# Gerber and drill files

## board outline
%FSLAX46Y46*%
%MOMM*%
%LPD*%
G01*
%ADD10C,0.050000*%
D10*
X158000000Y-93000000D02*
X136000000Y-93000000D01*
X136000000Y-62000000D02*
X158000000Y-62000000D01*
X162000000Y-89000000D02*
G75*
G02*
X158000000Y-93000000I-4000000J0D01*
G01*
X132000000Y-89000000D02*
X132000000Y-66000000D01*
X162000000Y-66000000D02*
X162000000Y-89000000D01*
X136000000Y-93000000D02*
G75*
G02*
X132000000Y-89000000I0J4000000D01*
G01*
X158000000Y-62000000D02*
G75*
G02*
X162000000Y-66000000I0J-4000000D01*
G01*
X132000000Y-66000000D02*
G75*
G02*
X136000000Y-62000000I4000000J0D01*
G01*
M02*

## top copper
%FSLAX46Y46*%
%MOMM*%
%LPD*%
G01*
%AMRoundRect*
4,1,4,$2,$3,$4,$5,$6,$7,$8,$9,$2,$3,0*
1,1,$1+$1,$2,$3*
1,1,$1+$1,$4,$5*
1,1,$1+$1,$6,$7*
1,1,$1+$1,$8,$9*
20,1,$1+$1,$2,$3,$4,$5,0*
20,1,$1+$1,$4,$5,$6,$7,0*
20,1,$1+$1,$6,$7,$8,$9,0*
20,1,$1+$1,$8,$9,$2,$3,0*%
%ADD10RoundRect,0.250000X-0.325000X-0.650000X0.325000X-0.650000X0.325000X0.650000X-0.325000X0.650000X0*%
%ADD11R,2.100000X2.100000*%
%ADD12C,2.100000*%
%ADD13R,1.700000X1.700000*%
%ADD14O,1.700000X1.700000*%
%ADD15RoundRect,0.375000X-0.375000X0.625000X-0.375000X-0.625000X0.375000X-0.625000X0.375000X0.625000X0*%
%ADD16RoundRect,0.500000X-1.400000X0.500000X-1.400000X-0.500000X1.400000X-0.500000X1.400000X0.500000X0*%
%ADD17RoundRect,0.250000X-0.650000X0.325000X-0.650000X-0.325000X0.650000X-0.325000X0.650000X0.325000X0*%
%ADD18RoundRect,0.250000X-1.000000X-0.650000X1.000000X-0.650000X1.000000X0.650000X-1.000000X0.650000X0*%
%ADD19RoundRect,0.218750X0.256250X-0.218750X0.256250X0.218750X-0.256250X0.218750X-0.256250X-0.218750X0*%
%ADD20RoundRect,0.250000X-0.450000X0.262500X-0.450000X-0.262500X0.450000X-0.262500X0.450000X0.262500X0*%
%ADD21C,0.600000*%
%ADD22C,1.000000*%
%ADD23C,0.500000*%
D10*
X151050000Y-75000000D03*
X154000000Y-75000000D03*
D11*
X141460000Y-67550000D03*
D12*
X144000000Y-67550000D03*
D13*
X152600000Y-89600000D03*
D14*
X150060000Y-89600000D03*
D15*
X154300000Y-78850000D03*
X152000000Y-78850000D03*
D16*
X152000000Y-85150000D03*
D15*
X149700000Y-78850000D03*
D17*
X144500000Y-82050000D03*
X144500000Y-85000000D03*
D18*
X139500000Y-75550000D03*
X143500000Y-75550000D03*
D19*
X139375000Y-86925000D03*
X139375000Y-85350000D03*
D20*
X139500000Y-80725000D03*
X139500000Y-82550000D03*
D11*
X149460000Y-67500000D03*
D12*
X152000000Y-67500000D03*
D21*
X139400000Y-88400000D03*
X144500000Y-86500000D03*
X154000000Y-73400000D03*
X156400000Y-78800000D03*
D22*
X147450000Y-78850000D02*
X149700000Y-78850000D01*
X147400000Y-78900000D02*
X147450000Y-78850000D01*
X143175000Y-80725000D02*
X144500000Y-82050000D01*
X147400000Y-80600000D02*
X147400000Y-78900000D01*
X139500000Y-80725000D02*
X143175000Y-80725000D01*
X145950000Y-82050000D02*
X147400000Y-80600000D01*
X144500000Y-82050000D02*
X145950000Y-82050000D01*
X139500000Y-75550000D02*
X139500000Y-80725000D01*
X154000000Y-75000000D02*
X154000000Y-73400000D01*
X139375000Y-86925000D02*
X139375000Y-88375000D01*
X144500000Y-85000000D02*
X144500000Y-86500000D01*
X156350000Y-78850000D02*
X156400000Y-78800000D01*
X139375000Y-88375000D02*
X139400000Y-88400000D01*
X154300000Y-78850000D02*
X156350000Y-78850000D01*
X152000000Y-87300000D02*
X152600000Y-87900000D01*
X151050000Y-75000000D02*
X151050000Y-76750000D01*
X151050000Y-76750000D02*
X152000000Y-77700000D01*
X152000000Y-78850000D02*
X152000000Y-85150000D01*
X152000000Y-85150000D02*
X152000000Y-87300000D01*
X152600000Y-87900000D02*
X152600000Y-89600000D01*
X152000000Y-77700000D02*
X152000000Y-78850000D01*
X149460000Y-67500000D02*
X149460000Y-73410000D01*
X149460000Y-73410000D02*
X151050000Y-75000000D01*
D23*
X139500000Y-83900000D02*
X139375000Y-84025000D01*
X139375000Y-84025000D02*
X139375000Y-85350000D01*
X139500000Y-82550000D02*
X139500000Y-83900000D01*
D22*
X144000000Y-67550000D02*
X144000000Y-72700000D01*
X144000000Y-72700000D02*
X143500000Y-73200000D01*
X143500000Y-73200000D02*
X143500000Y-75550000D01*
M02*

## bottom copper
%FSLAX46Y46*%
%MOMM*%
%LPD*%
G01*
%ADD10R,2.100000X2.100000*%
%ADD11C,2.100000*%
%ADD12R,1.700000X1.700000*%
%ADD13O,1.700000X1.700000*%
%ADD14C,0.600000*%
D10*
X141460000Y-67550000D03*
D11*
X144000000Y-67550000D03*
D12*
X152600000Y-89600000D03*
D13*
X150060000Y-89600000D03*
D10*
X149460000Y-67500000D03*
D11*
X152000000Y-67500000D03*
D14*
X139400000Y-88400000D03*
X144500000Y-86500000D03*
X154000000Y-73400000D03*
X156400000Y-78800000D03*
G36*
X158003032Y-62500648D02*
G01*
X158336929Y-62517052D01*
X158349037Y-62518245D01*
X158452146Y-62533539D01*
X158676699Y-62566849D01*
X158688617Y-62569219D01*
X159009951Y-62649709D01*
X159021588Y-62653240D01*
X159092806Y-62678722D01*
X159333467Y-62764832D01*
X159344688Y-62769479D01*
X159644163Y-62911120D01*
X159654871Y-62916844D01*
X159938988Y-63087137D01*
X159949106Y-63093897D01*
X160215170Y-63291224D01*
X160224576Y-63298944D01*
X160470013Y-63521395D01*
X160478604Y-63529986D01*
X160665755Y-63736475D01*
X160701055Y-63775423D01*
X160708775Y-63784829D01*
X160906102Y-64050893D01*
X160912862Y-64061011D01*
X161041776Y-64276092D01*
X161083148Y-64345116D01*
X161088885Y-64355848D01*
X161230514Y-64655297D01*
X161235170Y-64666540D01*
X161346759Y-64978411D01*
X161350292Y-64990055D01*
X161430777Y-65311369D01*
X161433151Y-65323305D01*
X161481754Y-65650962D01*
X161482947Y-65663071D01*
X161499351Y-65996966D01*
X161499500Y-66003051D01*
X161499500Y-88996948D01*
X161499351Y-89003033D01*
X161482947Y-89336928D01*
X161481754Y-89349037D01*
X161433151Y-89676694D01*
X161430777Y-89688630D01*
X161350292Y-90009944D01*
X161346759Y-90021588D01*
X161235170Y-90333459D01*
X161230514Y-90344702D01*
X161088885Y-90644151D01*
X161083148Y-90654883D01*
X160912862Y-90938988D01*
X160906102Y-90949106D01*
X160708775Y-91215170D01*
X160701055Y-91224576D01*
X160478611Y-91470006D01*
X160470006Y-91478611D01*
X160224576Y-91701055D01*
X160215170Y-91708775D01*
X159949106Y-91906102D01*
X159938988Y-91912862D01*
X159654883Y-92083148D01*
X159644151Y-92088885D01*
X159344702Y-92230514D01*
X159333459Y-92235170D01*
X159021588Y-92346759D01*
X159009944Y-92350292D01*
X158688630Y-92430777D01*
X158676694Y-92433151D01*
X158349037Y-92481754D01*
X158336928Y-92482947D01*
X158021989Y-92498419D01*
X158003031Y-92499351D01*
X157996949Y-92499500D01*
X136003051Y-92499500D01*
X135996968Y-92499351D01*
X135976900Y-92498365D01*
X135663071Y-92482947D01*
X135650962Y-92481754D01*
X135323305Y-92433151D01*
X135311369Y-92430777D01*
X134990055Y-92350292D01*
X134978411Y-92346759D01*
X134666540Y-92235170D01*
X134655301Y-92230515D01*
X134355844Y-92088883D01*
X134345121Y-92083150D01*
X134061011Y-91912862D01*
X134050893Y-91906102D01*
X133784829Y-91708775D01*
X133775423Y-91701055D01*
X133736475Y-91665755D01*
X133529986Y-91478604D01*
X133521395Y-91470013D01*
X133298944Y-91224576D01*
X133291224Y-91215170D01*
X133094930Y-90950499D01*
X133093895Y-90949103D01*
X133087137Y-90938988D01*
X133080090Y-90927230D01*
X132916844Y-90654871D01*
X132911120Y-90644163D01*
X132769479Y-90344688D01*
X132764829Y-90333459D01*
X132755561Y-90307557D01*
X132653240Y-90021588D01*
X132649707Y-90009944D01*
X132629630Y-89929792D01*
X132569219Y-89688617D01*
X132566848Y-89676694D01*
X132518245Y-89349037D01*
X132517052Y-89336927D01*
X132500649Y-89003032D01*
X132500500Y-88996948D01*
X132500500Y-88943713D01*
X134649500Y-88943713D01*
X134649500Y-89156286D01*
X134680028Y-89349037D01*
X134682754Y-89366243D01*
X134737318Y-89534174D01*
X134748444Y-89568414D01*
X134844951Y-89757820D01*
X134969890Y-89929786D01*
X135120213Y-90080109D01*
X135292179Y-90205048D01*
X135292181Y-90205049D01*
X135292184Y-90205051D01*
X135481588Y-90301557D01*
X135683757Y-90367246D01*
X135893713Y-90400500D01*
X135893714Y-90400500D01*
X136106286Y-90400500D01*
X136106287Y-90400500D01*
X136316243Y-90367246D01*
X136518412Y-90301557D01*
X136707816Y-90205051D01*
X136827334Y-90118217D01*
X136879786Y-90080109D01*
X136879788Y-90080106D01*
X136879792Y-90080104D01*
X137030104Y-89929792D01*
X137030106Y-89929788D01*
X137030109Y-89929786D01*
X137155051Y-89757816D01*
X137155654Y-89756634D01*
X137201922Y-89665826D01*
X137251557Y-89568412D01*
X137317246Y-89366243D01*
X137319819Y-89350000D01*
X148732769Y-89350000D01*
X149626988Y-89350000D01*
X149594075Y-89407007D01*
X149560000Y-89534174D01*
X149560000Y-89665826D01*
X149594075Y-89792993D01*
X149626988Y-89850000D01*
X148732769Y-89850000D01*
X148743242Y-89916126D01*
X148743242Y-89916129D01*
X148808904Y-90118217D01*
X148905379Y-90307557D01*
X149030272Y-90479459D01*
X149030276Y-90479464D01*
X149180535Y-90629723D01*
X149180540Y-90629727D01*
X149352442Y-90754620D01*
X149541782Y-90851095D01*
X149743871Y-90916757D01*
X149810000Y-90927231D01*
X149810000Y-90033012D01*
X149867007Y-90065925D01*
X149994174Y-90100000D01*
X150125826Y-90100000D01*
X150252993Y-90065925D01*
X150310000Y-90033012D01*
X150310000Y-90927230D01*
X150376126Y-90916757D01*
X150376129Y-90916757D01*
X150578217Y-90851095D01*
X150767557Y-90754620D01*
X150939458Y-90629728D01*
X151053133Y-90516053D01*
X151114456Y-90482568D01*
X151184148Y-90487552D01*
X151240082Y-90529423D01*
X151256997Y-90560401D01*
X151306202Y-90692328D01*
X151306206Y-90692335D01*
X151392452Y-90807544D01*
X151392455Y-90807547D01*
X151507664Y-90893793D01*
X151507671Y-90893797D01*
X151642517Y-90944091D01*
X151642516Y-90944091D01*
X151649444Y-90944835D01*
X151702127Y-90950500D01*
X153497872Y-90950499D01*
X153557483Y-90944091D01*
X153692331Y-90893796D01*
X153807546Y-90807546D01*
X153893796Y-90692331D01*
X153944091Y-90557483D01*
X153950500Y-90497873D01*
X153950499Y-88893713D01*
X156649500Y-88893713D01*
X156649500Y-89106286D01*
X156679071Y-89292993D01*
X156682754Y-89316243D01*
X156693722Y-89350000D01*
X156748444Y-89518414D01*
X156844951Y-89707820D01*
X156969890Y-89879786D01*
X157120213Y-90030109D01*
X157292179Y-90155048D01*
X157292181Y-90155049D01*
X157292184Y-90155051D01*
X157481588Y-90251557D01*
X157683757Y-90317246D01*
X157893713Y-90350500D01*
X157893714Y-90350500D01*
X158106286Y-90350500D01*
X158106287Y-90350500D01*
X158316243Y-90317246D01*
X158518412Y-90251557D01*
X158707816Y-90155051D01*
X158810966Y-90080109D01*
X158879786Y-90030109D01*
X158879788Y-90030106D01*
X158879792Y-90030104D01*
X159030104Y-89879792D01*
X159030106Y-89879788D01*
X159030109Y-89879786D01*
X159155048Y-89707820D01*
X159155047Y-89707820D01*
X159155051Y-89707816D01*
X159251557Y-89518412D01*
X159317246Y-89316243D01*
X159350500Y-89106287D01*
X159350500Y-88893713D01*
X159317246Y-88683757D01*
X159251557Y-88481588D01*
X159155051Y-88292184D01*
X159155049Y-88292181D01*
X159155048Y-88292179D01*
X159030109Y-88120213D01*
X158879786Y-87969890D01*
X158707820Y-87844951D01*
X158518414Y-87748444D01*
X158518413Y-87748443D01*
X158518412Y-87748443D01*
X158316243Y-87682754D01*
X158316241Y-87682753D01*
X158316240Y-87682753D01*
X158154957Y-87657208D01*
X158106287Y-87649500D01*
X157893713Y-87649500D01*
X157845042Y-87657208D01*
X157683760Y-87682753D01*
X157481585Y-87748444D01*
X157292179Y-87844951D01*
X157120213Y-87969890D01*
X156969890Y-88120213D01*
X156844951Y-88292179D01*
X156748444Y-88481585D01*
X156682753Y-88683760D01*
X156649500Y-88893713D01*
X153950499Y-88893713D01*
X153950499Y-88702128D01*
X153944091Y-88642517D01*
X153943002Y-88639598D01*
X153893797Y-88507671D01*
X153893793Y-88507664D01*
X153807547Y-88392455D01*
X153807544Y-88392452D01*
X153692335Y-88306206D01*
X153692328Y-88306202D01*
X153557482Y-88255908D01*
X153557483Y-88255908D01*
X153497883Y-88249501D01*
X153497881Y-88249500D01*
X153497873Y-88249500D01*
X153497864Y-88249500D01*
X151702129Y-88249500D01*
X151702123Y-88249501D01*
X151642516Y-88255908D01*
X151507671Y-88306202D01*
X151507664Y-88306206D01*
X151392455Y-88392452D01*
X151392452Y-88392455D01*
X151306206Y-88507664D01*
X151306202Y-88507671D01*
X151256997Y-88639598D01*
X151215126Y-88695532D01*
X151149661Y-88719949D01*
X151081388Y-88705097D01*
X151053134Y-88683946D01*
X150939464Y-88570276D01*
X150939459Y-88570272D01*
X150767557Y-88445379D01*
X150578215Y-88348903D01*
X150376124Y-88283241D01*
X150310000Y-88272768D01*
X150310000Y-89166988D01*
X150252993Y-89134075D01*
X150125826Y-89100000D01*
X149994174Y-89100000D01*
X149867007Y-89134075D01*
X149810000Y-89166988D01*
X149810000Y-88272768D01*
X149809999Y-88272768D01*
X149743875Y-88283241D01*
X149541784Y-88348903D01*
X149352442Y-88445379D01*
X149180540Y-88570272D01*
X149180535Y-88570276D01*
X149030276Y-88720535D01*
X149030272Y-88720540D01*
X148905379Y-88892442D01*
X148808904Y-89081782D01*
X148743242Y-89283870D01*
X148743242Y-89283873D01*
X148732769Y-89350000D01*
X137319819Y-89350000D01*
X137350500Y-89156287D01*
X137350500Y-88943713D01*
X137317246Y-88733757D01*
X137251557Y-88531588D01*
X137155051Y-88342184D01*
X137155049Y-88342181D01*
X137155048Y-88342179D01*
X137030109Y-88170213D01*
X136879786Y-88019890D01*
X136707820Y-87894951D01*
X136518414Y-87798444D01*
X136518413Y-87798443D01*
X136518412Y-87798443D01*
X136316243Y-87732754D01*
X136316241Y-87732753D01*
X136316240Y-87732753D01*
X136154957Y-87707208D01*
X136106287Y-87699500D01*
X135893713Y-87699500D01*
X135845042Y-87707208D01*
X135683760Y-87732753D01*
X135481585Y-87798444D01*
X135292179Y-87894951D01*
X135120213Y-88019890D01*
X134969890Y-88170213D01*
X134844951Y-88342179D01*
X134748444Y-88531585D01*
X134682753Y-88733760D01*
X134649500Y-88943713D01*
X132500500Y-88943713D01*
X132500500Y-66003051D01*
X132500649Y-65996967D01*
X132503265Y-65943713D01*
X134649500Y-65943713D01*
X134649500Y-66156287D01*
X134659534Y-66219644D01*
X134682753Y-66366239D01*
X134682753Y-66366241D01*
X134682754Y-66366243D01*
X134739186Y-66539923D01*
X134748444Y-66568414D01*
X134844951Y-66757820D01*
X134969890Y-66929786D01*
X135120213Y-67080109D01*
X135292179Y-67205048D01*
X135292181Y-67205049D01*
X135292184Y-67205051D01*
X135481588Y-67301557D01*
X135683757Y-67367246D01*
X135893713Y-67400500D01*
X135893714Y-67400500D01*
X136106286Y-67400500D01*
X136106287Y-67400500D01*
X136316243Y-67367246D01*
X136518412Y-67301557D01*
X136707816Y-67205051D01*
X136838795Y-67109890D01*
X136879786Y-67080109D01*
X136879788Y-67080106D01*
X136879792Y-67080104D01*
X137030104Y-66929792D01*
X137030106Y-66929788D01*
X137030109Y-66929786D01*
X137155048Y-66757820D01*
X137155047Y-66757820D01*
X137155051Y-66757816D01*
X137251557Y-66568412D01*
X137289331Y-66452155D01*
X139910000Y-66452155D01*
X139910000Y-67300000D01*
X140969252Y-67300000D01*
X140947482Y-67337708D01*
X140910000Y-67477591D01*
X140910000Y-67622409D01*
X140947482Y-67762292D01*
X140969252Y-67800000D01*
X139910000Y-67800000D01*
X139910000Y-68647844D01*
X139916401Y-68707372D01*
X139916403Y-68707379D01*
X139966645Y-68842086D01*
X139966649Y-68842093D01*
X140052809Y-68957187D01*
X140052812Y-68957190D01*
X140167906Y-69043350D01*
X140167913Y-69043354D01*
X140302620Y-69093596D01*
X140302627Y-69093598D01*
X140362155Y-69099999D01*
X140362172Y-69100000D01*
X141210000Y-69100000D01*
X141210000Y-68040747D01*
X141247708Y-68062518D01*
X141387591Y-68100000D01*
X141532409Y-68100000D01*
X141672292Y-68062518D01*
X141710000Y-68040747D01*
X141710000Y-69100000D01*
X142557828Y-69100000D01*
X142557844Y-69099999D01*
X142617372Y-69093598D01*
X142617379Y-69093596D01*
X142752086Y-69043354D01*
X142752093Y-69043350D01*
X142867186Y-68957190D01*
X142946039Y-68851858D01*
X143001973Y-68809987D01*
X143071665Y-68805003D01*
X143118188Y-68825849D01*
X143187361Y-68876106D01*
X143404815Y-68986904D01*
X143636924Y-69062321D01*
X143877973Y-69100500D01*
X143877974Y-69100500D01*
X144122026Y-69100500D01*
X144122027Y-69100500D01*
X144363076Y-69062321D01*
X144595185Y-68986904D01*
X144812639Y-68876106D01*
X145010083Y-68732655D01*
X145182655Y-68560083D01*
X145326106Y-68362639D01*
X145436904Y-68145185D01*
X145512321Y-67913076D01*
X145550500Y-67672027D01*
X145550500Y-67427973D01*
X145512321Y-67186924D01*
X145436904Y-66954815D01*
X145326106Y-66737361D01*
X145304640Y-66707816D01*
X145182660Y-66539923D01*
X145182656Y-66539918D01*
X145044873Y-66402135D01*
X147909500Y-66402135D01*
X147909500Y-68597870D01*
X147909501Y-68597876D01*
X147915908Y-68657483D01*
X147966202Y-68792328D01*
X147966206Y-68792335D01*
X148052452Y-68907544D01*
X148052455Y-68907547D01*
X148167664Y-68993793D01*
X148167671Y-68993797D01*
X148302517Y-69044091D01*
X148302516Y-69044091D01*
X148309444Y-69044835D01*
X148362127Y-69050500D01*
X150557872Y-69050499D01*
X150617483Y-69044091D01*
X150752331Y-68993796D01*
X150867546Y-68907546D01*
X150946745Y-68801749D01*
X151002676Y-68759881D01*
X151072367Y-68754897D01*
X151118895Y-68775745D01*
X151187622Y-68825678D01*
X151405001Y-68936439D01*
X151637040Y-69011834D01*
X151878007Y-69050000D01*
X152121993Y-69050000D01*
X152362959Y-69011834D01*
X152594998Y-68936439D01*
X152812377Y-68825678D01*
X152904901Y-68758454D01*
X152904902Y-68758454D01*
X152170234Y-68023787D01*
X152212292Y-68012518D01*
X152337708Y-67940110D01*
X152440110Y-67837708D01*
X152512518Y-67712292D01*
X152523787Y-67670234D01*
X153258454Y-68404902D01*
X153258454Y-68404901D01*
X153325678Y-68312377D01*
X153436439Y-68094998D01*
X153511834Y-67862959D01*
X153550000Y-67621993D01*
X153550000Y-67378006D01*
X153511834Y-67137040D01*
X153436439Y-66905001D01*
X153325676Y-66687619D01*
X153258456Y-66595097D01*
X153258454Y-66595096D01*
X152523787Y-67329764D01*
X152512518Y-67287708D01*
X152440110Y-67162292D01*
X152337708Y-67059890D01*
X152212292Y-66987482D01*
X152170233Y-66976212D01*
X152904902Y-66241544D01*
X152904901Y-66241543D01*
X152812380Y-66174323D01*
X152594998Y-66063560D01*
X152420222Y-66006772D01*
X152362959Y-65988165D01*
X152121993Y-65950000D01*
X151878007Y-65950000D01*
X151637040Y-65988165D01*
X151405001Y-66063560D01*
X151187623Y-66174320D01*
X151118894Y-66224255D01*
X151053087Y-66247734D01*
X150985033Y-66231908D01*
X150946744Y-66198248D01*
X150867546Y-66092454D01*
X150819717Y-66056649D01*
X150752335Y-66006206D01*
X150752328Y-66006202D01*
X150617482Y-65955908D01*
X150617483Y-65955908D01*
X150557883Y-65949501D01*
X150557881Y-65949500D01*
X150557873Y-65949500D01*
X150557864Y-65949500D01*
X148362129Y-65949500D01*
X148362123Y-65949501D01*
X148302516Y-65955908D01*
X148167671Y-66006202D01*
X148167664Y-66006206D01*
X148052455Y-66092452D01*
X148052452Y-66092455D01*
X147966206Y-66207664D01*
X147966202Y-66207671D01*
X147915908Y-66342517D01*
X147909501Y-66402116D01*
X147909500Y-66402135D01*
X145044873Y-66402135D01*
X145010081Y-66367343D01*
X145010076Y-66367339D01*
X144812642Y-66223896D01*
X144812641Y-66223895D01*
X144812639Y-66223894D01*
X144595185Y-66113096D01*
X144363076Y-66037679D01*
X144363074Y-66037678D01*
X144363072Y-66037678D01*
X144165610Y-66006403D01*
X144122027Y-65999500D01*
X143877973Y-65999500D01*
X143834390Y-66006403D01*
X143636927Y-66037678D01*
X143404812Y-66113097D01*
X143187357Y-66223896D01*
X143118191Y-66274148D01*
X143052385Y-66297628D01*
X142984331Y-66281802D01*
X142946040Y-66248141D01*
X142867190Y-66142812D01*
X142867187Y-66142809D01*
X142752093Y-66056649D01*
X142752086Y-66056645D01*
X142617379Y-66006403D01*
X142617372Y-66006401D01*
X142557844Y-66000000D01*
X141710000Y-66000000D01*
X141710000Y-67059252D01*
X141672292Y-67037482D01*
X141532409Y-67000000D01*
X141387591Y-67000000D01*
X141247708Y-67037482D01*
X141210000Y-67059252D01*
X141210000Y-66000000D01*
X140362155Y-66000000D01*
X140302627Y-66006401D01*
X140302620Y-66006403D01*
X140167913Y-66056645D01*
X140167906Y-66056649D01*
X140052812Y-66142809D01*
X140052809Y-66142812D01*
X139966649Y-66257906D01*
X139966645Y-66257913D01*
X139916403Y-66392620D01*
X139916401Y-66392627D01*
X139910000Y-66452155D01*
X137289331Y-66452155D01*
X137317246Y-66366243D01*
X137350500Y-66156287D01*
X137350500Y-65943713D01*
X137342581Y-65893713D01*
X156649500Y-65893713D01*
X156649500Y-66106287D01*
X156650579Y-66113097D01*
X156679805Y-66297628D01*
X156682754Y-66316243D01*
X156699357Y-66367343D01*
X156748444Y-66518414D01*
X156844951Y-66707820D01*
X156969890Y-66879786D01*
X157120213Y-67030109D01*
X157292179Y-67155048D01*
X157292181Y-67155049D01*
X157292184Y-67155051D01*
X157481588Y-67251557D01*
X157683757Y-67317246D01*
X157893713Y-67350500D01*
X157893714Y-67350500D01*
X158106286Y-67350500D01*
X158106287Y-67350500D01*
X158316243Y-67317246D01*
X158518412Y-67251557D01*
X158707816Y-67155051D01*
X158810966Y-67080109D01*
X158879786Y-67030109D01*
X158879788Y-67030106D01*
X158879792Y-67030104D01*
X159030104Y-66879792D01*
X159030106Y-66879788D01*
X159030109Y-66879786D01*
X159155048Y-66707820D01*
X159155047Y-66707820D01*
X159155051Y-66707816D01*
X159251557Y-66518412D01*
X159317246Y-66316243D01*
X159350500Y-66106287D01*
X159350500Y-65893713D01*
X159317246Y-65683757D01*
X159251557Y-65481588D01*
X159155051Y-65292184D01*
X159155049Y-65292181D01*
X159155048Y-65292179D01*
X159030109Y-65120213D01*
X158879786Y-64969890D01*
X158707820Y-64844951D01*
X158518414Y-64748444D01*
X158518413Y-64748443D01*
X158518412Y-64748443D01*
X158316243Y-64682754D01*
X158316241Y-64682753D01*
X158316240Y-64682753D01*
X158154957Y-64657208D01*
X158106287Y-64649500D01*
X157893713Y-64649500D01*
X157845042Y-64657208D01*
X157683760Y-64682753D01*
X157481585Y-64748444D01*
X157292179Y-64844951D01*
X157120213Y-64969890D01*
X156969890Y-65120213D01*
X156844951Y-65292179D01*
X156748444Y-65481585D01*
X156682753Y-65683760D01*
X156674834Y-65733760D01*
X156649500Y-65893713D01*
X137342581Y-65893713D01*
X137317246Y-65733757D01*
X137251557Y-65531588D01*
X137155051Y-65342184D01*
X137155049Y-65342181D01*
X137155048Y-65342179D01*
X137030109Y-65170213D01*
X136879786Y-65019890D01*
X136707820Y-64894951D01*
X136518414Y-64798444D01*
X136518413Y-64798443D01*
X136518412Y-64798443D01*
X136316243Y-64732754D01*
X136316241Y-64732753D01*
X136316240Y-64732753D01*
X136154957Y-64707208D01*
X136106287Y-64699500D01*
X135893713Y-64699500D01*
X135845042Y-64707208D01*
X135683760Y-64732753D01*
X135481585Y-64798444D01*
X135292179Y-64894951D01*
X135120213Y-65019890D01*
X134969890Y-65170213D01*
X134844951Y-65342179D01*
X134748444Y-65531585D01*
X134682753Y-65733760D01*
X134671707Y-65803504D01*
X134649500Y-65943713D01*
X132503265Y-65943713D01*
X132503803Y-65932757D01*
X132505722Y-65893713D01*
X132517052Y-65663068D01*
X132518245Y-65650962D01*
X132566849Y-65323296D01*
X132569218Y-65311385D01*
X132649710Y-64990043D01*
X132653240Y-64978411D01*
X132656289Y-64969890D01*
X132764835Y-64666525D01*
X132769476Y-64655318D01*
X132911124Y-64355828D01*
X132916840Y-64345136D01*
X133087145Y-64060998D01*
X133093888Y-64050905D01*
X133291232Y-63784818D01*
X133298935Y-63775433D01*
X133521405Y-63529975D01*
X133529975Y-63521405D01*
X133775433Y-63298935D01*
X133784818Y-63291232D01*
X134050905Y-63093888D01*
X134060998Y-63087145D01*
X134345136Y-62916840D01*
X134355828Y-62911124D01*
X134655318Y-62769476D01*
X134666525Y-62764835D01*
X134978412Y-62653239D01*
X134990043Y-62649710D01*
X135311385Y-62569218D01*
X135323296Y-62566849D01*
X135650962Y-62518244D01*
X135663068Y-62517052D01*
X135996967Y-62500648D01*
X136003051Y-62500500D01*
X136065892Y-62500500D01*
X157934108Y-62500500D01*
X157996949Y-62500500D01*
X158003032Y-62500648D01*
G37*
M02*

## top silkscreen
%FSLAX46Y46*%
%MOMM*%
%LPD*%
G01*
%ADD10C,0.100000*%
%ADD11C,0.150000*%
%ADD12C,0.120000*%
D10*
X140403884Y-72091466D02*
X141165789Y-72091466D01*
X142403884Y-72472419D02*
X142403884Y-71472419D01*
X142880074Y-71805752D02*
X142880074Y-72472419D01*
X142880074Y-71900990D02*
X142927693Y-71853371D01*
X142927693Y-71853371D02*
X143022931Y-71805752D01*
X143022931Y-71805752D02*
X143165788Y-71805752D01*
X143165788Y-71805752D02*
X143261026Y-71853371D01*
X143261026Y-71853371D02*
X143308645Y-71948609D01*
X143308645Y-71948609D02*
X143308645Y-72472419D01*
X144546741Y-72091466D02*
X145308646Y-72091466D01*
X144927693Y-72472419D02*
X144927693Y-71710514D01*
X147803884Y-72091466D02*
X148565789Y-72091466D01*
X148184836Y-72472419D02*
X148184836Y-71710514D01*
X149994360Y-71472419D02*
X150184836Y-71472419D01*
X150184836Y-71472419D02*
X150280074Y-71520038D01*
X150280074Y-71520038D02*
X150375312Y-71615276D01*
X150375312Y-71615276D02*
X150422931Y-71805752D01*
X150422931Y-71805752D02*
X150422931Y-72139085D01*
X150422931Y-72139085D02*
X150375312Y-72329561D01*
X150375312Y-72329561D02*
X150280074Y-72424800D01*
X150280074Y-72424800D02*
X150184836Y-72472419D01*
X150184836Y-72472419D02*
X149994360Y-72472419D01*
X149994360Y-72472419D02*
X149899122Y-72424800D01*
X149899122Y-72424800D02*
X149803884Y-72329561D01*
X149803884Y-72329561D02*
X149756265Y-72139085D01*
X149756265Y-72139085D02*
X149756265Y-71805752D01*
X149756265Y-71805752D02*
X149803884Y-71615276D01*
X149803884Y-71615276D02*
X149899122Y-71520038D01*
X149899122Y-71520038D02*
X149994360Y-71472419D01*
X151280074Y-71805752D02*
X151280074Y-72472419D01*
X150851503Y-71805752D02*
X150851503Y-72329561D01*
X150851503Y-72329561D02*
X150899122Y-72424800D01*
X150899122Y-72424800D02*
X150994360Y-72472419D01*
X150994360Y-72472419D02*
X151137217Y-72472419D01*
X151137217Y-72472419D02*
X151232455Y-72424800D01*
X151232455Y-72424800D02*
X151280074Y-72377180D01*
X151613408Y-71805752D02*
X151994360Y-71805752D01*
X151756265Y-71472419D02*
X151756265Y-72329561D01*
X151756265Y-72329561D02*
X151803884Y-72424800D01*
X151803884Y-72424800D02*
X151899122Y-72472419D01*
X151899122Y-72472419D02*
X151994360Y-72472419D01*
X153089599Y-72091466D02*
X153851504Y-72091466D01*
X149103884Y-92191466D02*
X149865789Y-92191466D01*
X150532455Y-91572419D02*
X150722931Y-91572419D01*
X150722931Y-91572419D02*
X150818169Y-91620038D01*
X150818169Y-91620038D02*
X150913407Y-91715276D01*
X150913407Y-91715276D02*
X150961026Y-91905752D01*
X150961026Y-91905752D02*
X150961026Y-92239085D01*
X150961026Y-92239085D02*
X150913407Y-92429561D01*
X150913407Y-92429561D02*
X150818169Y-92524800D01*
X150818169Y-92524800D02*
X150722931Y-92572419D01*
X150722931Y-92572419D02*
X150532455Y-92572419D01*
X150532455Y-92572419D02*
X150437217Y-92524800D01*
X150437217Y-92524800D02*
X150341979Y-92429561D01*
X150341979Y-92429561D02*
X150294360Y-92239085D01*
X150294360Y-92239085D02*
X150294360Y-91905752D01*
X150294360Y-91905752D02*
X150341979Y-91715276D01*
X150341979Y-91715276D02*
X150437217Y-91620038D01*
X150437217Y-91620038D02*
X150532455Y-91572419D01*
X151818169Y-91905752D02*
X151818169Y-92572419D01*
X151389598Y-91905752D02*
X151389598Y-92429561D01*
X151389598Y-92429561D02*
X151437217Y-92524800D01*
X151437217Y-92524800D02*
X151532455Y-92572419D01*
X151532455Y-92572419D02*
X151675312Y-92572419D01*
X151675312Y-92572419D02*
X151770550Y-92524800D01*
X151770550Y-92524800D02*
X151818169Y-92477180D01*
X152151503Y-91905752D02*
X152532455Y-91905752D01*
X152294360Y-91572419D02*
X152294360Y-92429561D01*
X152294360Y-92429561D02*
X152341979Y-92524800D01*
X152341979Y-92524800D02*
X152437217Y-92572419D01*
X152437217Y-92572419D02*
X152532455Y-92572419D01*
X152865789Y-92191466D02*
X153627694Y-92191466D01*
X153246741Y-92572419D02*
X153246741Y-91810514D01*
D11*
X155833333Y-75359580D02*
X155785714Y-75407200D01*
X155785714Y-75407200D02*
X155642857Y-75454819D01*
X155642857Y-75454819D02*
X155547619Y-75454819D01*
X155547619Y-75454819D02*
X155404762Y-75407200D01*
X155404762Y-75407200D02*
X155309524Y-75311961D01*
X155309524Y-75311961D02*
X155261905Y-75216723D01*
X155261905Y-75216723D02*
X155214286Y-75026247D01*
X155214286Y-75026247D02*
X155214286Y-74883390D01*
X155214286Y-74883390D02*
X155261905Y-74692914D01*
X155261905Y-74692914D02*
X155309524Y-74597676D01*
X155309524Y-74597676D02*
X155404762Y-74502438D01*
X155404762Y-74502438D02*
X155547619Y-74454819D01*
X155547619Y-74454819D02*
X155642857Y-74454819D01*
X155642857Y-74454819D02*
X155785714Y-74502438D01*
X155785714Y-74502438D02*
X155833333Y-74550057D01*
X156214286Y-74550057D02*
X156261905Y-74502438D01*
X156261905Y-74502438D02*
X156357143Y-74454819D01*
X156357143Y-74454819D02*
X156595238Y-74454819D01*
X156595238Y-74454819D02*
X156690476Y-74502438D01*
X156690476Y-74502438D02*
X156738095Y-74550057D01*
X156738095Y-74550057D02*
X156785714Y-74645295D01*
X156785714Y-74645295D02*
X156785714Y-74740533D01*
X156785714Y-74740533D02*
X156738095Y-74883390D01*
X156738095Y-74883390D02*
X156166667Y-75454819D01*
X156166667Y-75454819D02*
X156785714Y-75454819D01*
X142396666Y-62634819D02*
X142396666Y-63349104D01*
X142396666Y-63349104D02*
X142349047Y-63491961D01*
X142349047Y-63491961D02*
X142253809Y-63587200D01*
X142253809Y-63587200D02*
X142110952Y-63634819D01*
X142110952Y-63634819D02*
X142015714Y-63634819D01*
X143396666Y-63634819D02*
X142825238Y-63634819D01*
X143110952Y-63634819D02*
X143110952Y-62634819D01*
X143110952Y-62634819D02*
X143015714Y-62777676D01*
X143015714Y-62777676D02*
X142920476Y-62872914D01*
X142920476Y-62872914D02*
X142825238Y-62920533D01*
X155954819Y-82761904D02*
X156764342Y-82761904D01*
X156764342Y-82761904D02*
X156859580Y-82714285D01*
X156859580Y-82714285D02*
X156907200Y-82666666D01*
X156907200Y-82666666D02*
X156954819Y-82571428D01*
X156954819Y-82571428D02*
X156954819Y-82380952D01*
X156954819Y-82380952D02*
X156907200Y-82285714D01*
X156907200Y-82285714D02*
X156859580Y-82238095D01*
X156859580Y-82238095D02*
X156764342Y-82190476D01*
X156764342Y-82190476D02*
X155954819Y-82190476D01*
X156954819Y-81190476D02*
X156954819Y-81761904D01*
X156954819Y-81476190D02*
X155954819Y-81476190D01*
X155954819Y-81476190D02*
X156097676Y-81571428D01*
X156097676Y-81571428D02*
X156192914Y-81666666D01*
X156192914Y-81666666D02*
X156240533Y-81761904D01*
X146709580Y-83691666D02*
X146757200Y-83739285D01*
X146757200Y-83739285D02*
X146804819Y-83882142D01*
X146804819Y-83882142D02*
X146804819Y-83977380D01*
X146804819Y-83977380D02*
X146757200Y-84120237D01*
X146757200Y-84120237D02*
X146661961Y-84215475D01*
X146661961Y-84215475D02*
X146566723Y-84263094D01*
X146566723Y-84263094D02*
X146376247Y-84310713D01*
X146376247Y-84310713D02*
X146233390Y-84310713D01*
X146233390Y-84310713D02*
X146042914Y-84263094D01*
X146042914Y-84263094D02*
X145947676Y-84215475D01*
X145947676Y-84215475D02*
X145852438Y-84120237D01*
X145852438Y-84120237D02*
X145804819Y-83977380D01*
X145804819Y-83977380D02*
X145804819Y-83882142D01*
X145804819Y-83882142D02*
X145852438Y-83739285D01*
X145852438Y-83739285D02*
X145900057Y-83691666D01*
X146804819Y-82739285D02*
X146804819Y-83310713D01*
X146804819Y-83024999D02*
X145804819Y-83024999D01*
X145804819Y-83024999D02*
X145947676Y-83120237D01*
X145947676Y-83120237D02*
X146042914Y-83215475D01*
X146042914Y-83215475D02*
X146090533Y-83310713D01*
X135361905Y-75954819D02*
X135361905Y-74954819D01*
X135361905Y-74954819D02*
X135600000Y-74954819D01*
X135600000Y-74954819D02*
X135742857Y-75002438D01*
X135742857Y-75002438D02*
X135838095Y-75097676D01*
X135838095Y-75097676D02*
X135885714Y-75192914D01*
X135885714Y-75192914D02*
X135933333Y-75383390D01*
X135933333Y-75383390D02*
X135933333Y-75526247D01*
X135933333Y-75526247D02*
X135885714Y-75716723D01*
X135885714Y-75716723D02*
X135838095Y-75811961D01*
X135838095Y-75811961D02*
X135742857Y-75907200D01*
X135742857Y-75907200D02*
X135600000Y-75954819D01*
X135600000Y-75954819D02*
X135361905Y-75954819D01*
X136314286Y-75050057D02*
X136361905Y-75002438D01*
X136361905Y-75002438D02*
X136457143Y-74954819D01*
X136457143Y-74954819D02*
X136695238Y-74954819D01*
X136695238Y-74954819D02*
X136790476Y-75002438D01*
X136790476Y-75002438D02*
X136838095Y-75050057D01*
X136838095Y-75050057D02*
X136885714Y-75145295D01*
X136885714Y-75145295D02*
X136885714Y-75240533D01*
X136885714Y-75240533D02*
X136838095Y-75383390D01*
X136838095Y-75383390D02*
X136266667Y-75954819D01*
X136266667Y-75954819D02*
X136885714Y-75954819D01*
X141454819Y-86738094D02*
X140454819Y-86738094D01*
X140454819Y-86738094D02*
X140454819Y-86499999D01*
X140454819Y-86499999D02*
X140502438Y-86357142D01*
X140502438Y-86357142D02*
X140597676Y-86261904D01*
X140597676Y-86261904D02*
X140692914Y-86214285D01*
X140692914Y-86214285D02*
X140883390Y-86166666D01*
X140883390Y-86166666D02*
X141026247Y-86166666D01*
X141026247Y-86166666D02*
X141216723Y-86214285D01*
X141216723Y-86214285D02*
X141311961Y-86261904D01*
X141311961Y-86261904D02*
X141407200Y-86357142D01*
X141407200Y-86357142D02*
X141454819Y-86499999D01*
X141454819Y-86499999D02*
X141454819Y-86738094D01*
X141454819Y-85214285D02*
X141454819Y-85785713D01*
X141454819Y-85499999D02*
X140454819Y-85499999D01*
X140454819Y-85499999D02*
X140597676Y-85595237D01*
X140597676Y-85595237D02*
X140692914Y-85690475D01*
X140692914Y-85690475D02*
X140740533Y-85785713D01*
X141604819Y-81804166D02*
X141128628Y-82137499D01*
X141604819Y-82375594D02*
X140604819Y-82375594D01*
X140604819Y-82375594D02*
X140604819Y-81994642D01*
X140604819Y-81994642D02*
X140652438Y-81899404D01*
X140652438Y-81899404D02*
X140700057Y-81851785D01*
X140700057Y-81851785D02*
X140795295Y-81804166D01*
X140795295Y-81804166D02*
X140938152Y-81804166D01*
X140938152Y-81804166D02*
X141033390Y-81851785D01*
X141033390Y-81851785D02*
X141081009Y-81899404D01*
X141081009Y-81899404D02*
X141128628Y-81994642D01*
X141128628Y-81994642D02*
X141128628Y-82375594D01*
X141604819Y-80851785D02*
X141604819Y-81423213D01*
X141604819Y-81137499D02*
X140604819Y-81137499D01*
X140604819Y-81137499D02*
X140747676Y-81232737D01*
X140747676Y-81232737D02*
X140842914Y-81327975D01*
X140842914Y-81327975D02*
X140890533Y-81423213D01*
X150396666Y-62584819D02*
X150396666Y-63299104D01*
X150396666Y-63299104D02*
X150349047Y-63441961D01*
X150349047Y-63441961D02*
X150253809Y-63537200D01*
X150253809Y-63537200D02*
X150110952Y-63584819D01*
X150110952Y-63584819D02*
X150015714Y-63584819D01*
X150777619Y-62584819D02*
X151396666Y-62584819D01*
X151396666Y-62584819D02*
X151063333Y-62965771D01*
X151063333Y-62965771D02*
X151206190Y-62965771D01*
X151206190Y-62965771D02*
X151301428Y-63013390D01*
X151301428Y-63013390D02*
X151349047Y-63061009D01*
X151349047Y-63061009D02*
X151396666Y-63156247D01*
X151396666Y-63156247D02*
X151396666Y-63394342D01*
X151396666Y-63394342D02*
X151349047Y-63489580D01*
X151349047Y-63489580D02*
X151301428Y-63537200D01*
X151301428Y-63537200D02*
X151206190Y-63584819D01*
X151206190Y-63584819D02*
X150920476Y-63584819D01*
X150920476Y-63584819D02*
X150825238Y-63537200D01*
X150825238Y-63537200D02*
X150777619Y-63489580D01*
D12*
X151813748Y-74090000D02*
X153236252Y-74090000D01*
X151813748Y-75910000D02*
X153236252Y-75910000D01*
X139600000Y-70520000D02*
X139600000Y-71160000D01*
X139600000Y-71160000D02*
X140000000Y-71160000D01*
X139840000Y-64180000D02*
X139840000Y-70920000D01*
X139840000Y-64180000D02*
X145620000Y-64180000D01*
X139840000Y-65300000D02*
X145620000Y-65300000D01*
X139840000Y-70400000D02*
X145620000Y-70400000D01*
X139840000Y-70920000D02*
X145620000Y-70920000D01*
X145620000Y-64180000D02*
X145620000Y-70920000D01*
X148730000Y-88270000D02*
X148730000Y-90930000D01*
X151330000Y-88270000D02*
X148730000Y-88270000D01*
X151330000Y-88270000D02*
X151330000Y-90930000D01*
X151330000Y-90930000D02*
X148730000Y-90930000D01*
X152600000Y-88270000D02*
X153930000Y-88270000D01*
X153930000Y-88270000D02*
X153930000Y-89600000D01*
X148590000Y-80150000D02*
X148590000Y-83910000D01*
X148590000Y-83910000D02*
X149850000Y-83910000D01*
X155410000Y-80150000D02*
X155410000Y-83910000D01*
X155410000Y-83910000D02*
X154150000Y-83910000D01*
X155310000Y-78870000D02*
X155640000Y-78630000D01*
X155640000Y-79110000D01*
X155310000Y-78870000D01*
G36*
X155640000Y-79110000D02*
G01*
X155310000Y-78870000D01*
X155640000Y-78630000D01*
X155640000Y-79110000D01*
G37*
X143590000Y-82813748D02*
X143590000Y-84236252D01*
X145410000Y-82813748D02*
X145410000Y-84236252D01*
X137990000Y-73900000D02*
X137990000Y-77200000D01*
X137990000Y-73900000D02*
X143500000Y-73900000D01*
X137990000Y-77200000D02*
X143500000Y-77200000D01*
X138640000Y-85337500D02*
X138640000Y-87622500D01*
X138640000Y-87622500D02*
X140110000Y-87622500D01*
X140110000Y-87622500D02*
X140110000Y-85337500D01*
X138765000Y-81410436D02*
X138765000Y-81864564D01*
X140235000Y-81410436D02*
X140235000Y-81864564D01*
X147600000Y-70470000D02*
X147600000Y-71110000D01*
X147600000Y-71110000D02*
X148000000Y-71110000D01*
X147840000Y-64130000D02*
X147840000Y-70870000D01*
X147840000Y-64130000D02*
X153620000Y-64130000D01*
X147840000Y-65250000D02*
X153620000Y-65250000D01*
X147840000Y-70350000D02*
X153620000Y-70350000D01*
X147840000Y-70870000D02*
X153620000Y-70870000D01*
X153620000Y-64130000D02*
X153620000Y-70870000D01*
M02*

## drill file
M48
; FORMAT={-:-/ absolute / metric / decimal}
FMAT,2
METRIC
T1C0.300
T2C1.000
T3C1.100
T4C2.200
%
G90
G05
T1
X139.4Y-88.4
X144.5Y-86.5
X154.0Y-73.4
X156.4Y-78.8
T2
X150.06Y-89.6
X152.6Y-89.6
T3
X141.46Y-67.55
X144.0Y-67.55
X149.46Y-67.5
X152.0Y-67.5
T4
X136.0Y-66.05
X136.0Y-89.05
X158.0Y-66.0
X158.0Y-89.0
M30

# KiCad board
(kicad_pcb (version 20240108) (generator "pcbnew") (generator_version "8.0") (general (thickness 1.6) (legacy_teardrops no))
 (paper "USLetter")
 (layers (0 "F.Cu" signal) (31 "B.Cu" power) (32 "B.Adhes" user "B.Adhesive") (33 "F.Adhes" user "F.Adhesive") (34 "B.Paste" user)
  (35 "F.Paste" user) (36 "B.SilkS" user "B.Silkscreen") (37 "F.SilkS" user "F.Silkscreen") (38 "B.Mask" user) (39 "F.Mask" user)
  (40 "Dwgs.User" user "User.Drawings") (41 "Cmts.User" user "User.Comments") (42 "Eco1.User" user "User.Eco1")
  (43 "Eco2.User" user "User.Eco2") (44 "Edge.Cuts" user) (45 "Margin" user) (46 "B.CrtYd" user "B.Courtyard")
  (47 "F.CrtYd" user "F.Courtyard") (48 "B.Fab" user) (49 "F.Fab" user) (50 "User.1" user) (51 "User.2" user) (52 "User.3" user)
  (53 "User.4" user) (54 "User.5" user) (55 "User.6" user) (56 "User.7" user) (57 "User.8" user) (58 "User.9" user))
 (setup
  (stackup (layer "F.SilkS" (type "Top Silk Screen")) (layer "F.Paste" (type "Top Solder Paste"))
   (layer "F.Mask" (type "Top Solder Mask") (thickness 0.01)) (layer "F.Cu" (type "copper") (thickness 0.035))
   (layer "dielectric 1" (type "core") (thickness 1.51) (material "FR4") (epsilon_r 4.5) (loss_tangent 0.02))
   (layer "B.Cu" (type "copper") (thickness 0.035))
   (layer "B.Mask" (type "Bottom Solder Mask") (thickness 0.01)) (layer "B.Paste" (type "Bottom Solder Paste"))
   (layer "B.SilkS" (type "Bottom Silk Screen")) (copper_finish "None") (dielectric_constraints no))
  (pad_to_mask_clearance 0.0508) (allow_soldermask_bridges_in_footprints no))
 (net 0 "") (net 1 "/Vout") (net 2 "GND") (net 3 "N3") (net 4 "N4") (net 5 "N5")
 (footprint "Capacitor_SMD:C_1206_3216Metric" (layer "F.Cu") (at 152.525 75)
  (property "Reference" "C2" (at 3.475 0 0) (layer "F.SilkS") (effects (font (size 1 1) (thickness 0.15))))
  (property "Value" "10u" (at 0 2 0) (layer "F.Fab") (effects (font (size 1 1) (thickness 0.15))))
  (fp_line (start -0.711252 -0.91) (end 0.711252 -0.91) (stroke (width 0.12) (type solid)) (layer "F.SilkS"))
  (fp_line (start -0.711252 0.91) (end 0.711252 0.91) (stroke (width 0.12) (type solid)) (layer "F.SilkS"))
  (pad "1" smd roundrect (at -1.475 0) (size 1.15 1.8) (layers "F.Cu" "F.Paste" "F.Mask") (roundrect_rratio 0.217391) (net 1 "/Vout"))
  (pad "2" smd roundrect (at 1.475 0) (size 1.15 1.8) (layers "F.Cu" "F.Paste" "F.Mask") (roundrect_rratio 0.217391) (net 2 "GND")))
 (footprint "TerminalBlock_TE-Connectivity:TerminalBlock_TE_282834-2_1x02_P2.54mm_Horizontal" (layer "F.Cu") (at 141.46 67.55)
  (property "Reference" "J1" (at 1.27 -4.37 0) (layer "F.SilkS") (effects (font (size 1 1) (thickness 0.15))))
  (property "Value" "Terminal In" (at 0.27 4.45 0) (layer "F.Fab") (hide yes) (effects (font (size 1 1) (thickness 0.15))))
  (fp_line (start -1.86 2.97) (end -1.86 3.61) (stroke (width 0.12) (type solid)) (layer "F.SilkS"))
  (fp_line (start -1.86 3.61) (end -1.46 3.61) (stroke (width 0.12) (type solid)) (layer "F.SilkS"))
  (fp_line (start -1.62 -3.37) (end -1.62 3.37) (stroke (width 0.12) (type solid)) (layer "F.SilkS"))
  (fp_line (start -1.62 -3.37) (end 4.16 -3.37) (stroke (width 0.12) (type solid)) (layer "F.SilkS"))
  (fp_line (start -1.62 -2.25) (end 4.16 -2.25) (stroke (width 0.12) (type solid)) (layer "F.SilkS"))
  (fp_line (start -1.62 2.85) (end 4.16 2.85) (stroke (width 0.12) (type solid)) (layer "F.SilkS"))
  (fp_line (start -1.62 3.37) (end 4.16 3.37) (stroke (width 0.12) (type solid)) (layer "F.SilkS"))
  (fp_line (start 4.16 -3.37) (end 4.16 3.37) (stroke (width 0.12) (type solid)) (layer "F.SilkS"))
  (pad "1" thru_hole rect (at 0 0) (size 2.1 2.1) (drill 1.1) (layers "*.Cu" "*.Mask") (remove_unused_layers no) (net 2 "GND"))
  (pad "2" thru_hole circle (at 2.54 0) (size 2.1 2.1) (drill 1.1) (layers "*.Cu" "*.Mask") (remove_unused_layers no) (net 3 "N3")))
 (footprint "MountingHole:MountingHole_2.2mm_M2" (layer "F.Cu") (at 136 89.05)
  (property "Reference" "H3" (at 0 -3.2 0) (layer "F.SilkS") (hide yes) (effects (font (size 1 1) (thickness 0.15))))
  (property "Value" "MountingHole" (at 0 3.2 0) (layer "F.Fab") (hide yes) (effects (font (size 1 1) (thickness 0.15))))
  (pad "" np_thru_hole circle (at 0 0) (size 2.2 2.2) (drill 2.2) (layers "*.Cu" "*.Mask")))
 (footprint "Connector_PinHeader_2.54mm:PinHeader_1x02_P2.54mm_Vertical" (layer "F.Cu") (at 152.6 89.6 -90)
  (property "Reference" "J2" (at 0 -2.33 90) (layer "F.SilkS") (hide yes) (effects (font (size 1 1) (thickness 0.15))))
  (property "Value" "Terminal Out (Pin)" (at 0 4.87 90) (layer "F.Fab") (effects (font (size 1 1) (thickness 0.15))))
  (fp_line (start -1.33 3.87) (end 1.33 3.87) (stroke (width 0.12) (type solid)) (layer "F.SilkS"))
  (fp_line (start -1.33 1.27) (end -1.33 3.87) (stroke (width 0.12) (type solid)) (layer "F.SilkS"))
  (fp_line (start -1.33 1.27) (end 1.33 1.27) (stroke (width 0.12) (type solid)) (layer "F.SilkS"))
  (fp_line (start 1.33 1.27) (end 1.33 3.87) (stroke (width 0.12) (type solid)) (layer "F.SilkS"))
  (fp_line (start -1.33 0) (end -1.33 -1.33) (stroke (width 0.12) (type solid)) (layer "F.SilkS"))
  (fp_line (start -1.33 -1.33) (end 0 -1.33) (stroke (width 0.12) (type solid)) (layer "F.SilkS"))
  (pad "1" thru_hole rect (at 0 0 270) (size 1.7 1.7) (drill 1) (layers "*.Cu" "*.Mask") (remove_unused_layers no) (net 1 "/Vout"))
  (pad "2" thru_hole oval (at 0 2.54 270) (size 1.7 1.7) (drill 1) (layers "*.Cu" "*.Mask") (remove_unused_layers no) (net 2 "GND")))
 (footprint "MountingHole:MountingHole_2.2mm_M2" (layer "F.Cu") (at 158 89)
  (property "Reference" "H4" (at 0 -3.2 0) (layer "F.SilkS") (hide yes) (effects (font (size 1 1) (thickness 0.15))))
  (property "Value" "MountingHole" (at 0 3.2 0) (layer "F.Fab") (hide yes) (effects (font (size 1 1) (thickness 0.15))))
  (pad "" np_thru_hole circle (at 0 0) (size 2.2 2.2) (drill 2.2) (layers "*.Cu" "*.Mask")))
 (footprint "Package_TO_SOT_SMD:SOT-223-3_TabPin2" (layer "F.Cu") (at 152 82 -90)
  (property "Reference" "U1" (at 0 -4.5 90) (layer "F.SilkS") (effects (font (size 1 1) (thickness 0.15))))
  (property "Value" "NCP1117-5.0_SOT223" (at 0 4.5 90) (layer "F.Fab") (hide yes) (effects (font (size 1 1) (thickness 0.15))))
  (fp_line (start -1.85 3.41) (end 1.91 3.41) (stroke (width 0.12) (type solid)) (layer "F.SilkS"))
  (fp_line (start 1.91 3.41) (end 1.91 2.15) (stroke (width 0.12) (type solid)) (layer "F.SilkS"))
  (fp_line (start -1.85 -3.41) (end 1.91 -3.41) (stroke (width 0.12) (type solid)) (layer "F.SilkS"))
  (fp_line (start 1.91 -3.41) (end 1.91 -2.15) (stroke (width 0.12) (type solid)) (layer "F.SilkS"))
  (fp_poly
   (pts (xy -3.13 -3.31) (xy -3.37 -3.64) (xy -2.89 -3.64) (xy -3.13 -3.31)) (stroke (width 0.12) (type solid)) (fill solid)
   (layer "F.SilkS"))
  (pad "1" smd roundrect (at -3.15 -2.3 270) (size 2 1.5) (layers "F.Cu" "F.Paste" "F.Mask") (roundrect_rratio 0.25) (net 2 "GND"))
  (pad "2" smd roundrect (at -3.15 0 270) (size 2 1.5) (layers "F.Cu" "F.Paste" "F.Mask") (roundrect_rratio 0.25) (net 1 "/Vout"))
  (pad "2" smd roundrect (at 3.15 0 270) (size 2 3.8) (layers "F.Cu" "F.Paste" "F.Mask") (roundrect_rratio 0.25) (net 1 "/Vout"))
  (pad "3" smd roundrect (at -3.15 2.3 270) (size 2 1.5) (layers "F.Cu" "F.Paste" "F.Mask") (roundrect_rratio 0.25) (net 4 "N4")))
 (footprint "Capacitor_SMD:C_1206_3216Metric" (layer "F.Cu") (at 144.5 83.525 -90)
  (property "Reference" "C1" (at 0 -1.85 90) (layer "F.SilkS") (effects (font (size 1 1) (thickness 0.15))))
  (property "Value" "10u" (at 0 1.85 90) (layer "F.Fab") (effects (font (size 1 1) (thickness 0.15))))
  (fp_line (start -0.711252 0.91) (end 0.711252 0.91) (stroke (width 0.12) (type solid)) (layer "F.SilkS"))
  (fp_line (start -0.711252 -0.91) (end 0.711252 -0.91) (stroke (width 0.12) (type solid)) (layer "F.SilkS"))
  (pad "1" smd roundrect (at -1.475 0 270) (size 1.15 1.8) (layers "F.Cu" "F.Paste" "F.Mask") (roundrect_rratio 0.217391) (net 4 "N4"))
  (pad "2" smd roundrect (at 1.475 0 270) (size 1.15 1.8) (layers "F.Cu" "F.Paste" "F.Mask") (roundrect_rratio 0.217391) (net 2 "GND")))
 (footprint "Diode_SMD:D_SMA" (layer "F.Cu") (at 141.5 75.55)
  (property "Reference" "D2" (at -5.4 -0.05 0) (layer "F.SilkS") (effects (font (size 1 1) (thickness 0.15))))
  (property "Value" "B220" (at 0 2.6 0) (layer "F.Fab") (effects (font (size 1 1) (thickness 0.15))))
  (fp_line (start -3.51 -1.65) (end -3.51 1.65) (stroke (width 0.12) (type solid)) (layer "F.SilkS"))
  (fp_line (start -3.51 -1.65) (end 2 -1.65) (stroke (width 0.12) (type solid)) (layer "F.SilkS"))
  (fp_line (start -3.51 1.65) (end 2 1.65) (stroke (width 0.12) (type solid)) (layer "F.SilkS"))
  (pad "1" smd roundrect (at -2 0) (size 2.5 1.8) (layers "F.Cu" "F.Paste" "F.Mask") (roundrect_rratio 0.1388888889) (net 4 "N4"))
  (pad "2" smd roundrect (at 2 0) (size 2.5 1.8) (layers "F.Cu" "F.Paste" "F.Mask") (roundrect_rratio 0.1388888889) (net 3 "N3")))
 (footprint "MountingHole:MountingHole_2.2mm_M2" (layer "F.Cu") (at 158 66)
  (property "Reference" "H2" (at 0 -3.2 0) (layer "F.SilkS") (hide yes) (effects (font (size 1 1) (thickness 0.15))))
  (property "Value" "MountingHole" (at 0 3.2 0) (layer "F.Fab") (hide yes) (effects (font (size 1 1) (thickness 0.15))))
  (pad "" np_thru_hole circle (at 0 0) (size 2.2 2.2) (drill 2.2) (layers "*.Cu" "*.Mask")))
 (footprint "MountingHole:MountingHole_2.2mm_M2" (layer "F.Cu") (at 136 66.05)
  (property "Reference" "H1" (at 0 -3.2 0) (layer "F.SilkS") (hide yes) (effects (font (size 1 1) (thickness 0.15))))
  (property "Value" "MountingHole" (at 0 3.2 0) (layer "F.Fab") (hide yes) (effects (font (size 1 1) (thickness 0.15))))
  (pad "" np_thru_hole circle (at 0 0) (size 2.2 2.2) (drill 2.2) (layers "*.Cu" "*.Mask")))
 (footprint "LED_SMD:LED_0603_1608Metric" (layer "F.Cu") (at 139.375 86.1375 90)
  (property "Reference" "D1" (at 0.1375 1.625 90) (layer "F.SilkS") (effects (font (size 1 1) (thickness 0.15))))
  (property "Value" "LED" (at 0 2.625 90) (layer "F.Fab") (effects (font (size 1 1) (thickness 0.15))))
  (fp_line (start 0.8 -0.735) (end -1.485 -0.735) (stroke (width 0.12) (type solid)) (layer "F.SilkS"))
  (fp_line (start -1.485 -0.735) (end -1.485 0.735) (stroke (width 0.12) (type solid)) (layer "F.SilkS"))
  (fp_line (start -1.485 0.735) (end 0.8 0.735) (stroke (width 0.12) (type solid)) (layer "F.SilkS"))
  (pad "1" smd roundrect (at -0.7875 0 90) (size 0.875 0.95) (layers "F.Cu" "F.Paste" "F.Mask") (roundrect_rratio 0.25) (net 2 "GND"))
  (pad "2" smd roundrect (at 0.7875 0 90) (size 0.875 0.95) (layers "F.Cu" "F.Paste" "F.Mask") (roundrect_rratio 0.25) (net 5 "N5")))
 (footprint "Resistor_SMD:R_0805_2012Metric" (layer "F.Cu") (at 139.5 81.6375 -90)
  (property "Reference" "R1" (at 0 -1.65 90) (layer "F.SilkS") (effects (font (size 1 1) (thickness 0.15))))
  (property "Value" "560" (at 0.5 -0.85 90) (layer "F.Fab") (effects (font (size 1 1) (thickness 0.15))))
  (fp_line (start -0.227064 0.735) (end 0.227064 0.735) (stroke (width 0.12) (type solid)) (layer "F.SilkS"))
  (fp_line (start -0.227064 -0.735) (end 0.227064 -0.735) (stroke (width 0.12) (type solid)) (layer "F.SilkS"))
  (pad "1" smd roundrect (at -0.9125 0 270) (size 1.025 1.4) (layers "F.Cu" "F.Paste" "F.Mask") (roundrect_rratio 0.243902) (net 4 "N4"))
  (pad "2" smd roundrect (at 0.9125 0 270) (size 1.025 1.4) (layers "F.Cu" "F.Paste" "F.Mask") (roundrect_rratio 0.243902) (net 5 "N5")))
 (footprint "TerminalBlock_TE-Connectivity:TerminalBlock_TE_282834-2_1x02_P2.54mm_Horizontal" (layer "F.Cu") (at 149.46 67.5)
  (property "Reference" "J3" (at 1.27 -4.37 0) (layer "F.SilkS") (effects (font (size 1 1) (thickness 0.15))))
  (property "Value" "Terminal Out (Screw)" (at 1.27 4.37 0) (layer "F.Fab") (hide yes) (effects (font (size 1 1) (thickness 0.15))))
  (fp_line (start -1.86 2.97) (end -1.86 3.61) (stroke (width 0.12) (type solid)) (layer "F.SilkS"))
  (fp_line (start -1.86 3.61) (end -1.46 3.61) (stroke (width 0.12) (type solid)) (layer "F.SilkS"))
  (fp_line (start -1.62 -3.37) (end -1.62 3.37) (stroke (width 0.12) (type solid)) (layer "F.SilkS"))
  (fp_line (start -1.62 -3.37) (end 4.16 -3.37) (stroke (width 0.12) (type solid)) (layer "F.SilkS"))
  (fp_line (start -1.62 -2.25) (end 4.16 -2.25) (stroke (width 0.12) (type solid)) (layer "F.SilkS"))
  (fp_line (start -1.62 2.85) (end 4.16 2.85) (stroke (width 0.12) (type solid)) (layer "F.SilkS"))
  (fp_line (start -1.62 3.37) (end 4.16 3.37) (stroke (width 0.12) (type solid)) (layer "F.SilkS"))
  (fp_line (start 4.16 -3.37) (end 4.16 3.37) (stroke (width 0.12) (type solid)) (layer "F.SilkS"))
  (pad "1" thru_hole rect (at 0 0) (size 2.1 2.1) (drill 1.1) (layers "*.Cu" "*.Mask") (remove_unused_layers no) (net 1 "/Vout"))
  (pad "2" thru_hole circle (at 2.54 0) (size 2.1 2.1) (drill 1.1) (layers "*.Cu" "*.Mask") (remove_unused_layers no) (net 2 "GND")))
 (gr_line (start 158 93) (end 136 93) (stroke (width 0.05) (type default)) (layer "Edge.Cuts"))
 (gr_line (start 136 62) (end 158 62) (stroke (width 0.05) (type default)) (layer "Edge.Cuts"))
 (gr_arc (start 162 89) (mid 160.828427 91.828427) (end 158 93) (stroke (width 0.05) (type default)) (layer "Edge.Cuts"))
 (gr_line (start 132 89) (end 132 66) (stroke (width 0.05) (type default)) (layer "Edge.Cuts"))
 (gr_line (start 162 66) (end 162 89) (stroke (width 0.05) (type default)) (layer "Edge.Cuts"))
 (gr_arc (start 136 93) (mid 133.171573 91.828427) (end 132 89) (stroke (width 0.05) (type default)) (layer "Edge.Cuts"))
 (gr_arc (start 158 62) (mid 160.828427 63.171573) (end 162 66) (stroke (width 0.05) (type default)) (layer "Edge.Cuts"))
 (gr_arc (start 132 66) (mid 133.171573 63.171573) (end 136 62) (stroke (width 0.05) (type default)) (layer "Edge.Cuts"))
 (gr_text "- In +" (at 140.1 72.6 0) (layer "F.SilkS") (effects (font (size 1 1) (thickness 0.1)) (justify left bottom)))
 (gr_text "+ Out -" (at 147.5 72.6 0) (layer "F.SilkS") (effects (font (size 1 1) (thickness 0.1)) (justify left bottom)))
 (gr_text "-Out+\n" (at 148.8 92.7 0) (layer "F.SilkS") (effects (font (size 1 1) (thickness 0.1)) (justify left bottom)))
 (segment (start 147.45 78.85) (end 149.7 78.85) (width 1) (layer "F.Cu") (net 4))
 (segment (start 147.4 78.9) (end 147.45 78.85) (width 1) (layer "F.Cu") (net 4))
 (segment (start 143.175 80.725) (end 144.5 82.05) (width 1) (layer "F.Cu") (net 4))
 (segment (start 147.4 80.6) (end 147.4 78.9) (width 1) (layer "F.Cu") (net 4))
 (segment (start 139.5 80.725) (end 143.175 80.725) (width 1) (layer "F.Cu") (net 4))
 (segment (start 145.95 82.05) (end 147.4 80.6) (width 1) (layer "F.Cu") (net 4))
 (segment (start 144.5 82.05) (end 145.95 82.05) (width 1) (layer "F.Cu") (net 4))
 (segment (start 139.5 75.55) (end 139.5 80.725) (width 1) (layer "F.Cu") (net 4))
 (segment (start 154 75) (end 154 73.4) (width 1) (layer "F.Cu") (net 2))
 (segment (start 139.375 86.925) (end 139.375 88.375) (width 1) (layer "F.Cu") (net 2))
 (segment (start 144.5 85) (end 144.5 86.5) (width 1) (layer "F.Cu") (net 2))
 (segment (start 156.35 78.85) (end 156.4 78.8) (width 1) (layer "F.Cu") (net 2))
 (segment (start 139.375 88.375) (end 139.4 88.4) (width 1) (layer "F.Cu") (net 2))
 (segment (start 154.3 78.85) (end 156.35 78.85) (width 1) (layer "F.Cu") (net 2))
 (via (at 139.4 88.4) (size 0.6) (drill 0.3) (layers "F.Cu" "B.Cu") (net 2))
 (via (at 144.5 86.5) (size 0.6) (drill 0.3) (layers "F.Cu" "B.Cu") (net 2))
 (via (at 154 73.4) (size 0.6) (drill 0.3) (layers "F.Cu" "B.Cu") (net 2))
 (via (at 156.4 78.8) (size 0.6) (drill 0.3) (layers "F.Cu" "B.Cu") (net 2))
 (segment (start 152 87.3) (end 152.6 87.9) (width 1) (layer "F.Cu") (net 1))
 (segment (start 151.05 75) (end 151.05 76.75) (width 1) (layer "F.Cu") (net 1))
 (segment (start 151.05 76.75) (end 152 77.7) (width 1) (layer "F.Cu") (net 1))
 (segment (start 152 78.85) (end 152 85.15) (width 1) (layer "F.Cu") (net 1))
 (segment (start 152 85.15) (end 152 87.3) (width 1) (layer "F.Cu") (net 1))
 (segment (start 152.6 87.9) (end 152.6 89.6) (width 1) (layer "F.Cu") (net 1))
 (segment (start 152 77.7) (end 152 78.85) (width 1) (layer "F.Cu") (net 1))
 (segment (start 149.46 67.5) (end 149.46 73.41) (width 1) (layer "F.Cu") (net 1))
 (segment (start 149.46 73.41) (end 151.05 75) (width 1) (layer "F.Cu") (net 1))
 (segment (start 139.5 83.9) (end 139.375 84.025) (width 0.5) (layer "F.Cu") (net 5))
 (segment (start 139.375 84.025) (end 139.375 85.35) (width 0.5) (layer "F.Cu") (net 5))
 (segment (start 139.5 82.55) (end 139.5 83.9) (width 0.5) (layer "F.Cu") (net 5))
 (segment (start 144 67.55) (end 144 72.7) (width 1) (layer "F.Cu") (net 3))
 (segment (start 144 72.7) (end 143.5 73.2) (width 1) (layer "F.Cu") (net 3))
 (segment (start 143.5 73.2) (end 143.5 75.55) (width 1) (layer "F.Cu") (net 3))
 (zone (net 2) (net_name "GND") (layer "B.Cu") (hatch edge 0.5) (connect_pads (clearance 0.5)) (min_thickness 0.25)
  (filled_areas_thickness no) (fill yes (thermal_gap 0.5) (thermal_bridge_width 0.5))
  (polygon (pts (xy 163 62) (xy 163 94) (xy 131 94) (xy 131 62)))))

